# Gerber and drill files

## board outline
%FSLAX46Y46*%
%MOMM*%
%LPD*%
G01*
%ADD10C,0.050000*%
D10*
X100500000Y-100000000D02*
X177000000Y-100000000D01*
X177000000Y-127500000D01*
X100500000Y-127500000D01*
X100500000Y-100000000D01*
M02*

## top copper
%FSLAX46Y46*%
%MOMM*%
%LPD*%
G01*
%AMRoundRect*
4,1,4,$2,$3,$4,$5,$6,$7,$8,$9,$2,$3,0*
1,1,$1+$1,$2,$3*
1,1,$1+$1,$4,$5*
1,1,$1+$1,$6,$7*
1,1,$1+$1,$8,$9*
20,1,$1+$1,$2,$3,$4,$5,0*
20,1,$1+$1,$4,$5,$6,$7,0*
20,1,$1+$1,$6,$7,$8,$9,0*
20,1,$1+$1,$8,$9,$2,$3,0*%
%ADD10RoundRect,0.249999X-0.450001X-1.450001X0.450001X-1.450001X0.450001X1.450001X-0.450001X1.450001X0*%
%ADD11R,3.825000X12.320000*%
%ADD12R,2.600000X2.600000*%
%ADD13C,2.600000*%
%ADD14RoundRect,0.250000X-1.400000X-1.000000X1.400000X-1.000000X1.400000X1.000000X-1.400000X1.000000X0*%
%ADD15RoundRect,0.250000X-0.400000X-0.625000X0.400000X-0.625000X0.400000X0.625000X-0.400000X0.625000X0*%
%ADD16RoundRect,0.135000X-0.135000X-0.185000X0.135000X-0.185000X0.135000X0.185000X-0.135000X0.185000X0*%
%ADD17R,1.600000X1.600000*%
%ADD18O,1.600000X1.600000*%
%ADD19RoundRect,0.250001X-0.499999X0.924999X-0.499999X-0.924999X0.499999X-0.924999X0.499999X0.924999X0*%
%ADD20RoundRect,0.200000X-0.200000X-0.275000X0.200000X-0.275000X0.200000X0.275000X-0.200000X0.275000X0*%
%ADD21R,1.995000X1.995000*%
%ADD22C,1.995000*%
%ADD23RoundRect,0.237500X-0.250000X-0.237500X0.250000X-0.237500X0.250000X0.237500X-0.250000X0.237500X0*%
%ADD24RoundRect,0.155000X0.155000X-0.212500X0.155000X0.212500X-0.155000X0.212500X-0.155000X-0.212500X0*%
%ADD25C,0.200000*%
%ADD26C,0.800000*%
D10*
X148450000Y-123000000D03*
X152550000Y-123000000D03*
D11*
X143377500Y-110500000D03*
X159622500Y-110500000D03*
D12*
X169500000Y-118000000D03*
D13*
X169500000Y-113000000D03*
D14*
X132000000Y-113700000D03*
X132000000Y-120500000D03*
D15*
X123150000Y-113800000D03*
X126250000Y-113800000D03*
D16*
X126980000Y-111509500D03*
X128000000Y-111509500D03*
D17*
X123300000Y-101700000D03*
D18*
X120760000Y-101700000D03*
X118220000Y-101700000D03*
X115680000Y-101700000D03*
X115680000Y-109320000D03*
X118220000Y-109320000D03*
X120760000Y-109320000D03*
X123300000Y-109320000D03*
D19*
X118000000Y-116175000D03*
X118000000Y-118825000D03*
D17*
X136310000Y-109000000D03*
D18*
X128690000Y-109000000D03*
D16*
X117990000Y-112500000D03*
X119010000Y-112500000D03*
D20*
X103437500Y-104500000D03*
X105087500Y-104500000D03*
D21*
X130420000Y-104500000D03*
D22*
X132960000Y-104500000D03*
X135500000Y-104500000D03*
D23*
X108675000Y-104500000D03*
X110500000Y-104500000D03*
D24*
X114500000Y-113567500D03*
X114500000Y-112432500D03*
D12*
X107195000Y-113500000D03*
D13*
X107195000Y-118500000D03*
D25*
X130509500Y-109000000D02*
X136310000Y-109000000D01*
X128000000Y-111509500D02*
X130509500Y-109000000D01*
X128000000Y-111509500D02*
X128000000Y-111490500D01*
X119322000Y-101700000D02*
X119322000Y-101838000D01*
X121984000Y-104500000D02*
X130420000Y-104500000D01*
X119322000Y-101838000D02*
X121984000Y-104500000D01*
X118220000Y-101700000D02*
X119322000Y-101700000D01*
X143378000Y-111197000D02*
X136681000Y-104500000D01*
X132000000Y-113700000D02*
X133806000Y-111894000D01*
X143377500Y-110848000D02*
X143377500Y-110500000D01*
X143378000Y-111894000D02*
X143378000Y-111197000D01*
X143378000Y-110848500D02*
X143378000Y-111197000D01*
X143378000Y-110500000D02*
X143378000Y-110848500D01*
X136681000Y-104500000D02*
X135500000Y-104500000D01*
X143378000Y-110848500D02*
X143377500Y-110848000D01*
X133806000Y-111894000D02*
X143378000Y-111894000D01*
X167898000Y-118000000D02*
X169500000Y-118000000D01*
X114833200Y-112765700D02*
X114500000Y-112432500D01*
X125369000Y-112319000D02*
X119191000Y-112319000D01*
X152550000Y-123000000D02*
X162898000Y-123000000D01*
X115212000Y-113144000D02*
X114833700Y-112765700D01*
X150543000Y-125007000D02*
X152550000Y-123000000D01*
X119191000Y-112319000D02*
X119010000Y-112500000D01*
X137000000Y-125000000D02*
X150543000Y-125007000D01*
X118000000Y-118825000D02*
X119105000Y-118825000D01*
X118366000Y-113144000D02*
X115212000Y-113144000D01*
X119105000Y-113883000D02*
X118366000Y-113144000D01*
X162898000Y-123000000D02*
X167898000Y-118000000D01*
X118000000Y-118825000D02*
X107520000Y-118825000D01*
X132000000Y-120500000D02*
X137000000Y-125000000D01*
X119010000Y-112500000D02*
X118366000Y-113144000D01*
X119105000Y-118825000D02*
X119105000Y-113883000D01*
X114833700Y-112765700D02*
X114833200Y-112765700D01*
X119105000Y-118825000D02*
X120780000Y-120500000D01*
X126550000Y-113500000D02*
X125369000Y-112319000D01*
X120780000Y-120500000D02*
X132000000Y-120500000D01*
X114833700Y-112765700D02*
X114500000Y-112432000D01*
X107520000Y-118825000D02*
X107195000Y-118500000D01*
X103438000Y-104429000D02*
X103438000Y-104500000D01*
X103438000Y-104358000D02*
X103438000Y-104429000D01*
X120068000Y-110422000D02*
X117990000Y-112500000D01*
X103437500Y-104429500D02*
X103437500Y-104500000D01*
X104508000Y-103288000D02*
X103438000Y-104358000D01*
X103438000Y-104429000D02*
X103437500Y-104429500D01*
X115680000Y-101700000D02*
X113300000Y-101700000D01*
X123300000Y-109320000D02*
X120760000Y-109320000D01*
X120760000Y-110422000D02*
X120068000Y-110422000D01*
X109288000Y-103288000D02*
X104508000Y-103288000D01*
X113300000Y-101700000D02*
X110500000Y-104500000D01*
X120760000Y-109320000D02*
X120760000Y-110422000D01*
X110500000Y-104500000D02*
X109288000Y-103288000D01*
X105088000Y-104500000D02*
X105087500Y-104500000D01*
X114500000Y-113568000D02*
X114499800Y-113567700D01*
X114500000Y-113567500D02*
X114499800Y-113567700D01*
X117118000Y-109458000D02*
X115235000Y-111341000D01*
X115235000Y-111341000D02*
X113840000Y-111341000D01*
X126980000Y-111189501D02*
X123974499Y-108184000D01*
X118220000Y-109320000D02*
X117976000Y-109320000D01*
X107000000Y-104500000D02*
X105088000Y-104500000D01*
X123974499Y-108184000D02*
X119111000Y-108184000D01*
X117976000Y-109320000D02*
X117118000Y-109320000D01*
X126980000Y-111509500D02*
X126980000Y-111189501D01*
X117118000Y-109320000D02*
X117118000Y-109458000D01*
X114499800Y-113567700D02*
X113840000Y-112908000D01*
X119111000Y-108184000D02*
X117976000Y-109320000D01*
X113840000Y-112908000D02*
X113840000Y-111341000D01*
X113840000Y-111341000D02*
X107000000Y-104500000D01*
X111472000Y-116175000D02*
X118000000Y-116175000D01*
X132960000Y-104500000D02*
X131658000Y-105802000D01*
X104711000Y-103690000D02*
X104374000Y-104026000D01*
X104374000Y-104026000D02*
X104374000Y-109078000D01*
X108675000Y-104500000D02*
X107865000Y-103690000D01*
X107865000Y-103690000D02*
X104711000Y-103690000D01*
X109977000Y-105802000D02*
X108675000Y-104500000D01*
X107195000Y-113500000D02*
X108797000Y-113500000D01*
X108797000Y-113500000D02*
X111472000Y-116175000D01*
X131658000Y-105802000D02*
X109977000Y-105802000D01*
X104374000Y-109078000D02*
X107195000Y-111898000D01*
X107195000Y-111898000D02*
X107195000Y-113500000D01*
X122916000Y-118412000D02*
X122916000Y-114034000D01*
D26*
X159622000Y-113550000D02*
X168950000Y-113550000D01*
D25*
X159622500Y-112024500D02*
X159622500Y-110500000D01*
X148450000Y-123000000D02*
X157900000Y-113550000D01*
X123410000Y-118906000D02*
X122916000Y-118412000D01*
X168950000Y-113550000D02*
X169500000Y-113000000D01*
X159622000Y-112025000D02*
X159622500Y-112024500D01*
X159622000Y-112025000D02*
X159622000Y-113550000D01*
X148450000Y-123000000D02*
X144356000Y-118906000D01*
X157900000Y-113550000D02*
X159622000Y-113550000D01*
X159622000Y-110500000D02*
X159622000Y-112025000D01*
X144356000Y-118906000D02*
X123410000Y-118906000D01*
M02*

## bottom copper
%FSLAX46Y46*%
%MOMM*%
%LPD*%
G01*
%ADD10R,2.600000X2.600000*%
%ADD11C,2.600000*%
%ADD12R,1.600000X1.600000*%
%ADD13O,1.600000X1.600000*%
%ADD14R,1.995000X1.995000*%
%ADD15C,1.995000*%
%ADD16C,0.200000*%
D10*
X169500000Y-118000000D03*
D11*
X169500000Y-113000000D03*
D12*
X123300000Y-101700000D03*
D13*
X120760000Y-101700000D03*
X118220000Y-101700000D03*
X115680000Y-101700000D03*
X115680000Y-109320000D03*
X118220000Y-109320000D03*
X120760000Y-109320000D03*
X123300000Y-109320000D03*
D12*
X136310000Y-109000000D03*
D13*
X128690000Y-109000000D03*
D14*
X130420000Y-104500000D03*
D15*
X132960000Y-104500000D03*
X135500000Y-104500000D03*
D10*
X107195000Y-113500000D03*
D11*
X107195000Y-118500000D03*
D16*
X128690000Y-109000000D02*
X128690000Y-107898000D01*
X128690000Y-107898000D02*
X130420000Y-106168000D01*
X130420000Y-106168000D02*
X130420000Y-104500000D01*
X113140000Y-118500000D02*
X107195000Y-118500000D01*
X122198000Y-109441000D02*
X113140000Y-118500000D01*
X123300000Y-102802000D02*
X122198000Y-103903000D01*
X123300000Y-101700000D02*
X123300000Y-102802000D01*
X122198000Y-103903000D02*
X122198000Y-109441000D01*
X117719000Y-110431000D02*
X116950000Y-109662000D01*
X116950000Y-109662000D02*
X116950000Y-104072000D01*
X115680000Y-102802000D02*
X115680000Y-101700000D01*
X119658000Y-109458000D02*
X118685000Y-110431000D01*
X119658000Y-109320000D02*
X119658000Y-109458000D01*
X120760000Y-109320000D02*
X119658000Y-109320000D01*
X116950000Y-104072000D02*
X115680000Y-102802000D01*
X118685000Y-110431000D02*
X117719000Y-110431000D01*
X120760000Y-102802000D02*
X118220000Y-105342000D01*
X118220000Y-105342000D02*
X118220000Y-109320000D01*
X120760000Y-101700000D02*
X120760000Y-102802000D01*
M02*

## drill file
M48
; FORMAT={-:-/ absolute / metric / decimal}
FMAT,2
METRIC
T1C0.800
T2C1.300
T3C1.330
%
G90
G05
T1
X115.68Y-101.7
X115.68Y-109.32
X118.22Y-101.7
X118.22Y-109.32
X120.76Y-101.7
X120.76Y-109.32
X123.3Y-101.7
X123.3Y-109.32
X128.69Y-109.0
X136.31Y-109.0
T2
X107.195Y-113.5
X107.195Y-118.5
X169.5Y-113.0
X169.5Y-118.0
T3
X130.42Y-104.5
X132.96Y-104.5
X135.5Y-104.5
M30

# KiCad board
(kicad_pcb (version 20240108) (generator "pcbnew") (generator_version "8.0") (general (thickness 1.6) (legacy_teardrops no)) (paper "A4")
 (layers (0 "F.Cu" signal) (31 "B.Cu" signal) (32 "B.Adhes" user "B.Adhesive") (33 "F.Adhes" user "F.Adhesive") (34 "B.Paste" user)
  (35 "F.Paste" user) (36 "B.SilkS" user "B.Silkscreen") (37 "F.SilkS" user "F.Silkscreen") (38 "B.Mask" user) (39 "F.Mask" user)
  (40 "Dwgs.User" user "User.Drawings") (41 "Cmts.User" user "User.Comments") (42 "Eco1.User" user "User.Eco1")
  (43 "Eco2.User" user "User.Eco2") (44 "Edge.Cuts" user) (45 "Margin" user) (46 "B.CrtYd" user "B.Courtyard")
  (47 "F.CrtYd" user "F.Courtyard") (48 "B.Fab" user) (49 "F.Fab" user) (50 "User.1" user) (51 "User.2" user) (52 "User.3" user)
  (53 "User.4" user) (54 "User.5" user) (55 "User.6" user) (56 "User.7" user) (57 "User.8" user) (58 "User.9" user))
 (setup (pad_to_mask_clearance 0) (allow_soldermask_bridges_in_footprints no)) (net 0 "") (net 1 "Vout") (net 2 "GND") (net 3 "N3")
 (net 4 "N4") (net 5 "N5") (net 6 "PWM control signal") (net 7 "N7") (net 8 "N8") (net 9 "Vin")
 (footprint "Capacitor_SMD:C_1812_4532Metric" (layer "F.Cu") (at 150.5 123)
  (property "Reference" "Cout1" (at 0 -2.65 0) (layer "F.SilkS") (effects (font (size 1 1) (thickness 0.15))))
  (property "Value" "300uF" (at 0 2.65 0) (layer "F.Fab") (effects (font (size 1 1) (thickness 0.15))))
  (pad "1" smd roundrect (at -2.05 0) (size 1.4 3.4) (layers "F.Cu" "F.Paste" "F.Mask") (roundrect_rratio 0.178571) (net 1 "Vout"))
  (pad "2" smd roundrect (at 2.05 0) (size 1.4 3.4) (layers "F.Cu" "F.Paste" "F.Mask") (roundrect_rratio 0.178571) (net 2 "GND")))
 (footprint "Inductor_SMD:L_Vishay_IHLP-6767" (layer "F.Cu") (at 151.5 110.5)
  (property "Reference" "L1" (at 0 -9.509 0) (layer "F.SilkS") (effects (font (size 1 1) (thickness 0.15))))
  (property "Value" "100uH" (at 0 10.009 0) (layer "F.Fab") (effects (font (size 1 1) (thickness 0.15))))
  (pad "1" smd rect (at -8.1225 0) (size 3.825 12.32) (layers "F.Cu" "F.Paste" "F.Mask") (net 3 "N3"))
  (pad "2" smd rect (at 8.1225 0) (size 3.825 12.32) (layers "F.Cu" "F.Paste" "F.Mask") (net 1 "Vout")))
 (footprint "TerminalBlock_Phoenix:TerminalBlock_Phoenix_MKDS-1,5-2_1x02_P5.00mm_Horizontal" (layer "F.Cu") (at 169.5 118 90)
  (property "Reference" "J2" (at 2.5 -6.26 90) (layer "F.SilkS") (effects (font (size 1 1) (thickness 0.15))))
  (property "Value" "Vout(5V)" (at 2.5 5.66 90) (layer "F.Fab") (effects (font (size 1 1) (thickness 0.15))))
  (pad "1" thru_hole rect (at 0 0 90) (size 2.6 2.6) (drill 1.3) (layers "*.Cu" "*.Mask") (remove_unused_layers no) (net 2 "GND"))
  (pad "2" thru_hole circle (at 5 0 90) (size 2.6 2.6) (drill 1.3) (layers "*.Cu" "*.Mask") (remove_unused_layers no) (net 1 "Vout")))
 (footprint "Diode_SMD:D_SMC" (layer "F.Cu") (at 132 117.1 -90)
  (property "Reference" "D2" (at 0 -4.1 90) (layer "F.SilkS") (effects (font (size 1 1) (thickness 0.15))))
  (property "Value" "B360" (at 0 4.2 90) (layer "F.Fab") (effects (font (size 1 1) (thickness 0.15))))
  (pad "1" smd roundrect (at -3.4 0) (size 3.3 2.5) (layers "F.Cu" "F.Paste" "F.Mask") (roundrect_rratio 0.1) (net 3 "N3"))
  (pad "2" smd roundrect (at 3.4 0) (size 3.3 2.5) (layers "F.Cu" "F.Paste" "F.Mask") (roundrect_rratio 0.1) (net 2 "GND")))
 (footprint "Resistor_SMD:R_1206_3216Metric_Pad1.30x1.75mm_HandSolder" (layer "F.Cu") (at 124.7 113.8)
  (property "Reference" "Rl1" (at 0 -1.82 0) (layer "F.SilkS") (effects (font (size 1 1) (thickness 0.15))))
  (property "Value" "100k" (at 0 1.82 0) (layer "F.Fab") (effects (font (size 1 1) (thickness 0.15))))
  (pad "1" smd roundrect (at -1.55 0) (size 1.3 1.75) (layers "F.Cu" "F.Paste" "F.Mask") (roundrect_rratio 0.192308) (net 1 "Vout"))
  (pad "2" smd roundrect (at 1.55 0) (size 1.3 1.75) (layers "F.Cu" "F.Paste" "F.Mask") (roundrect_rratio 0.192308) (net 2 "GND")))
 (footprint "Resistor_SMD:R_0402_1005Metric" (layer "F.Cu") (at 127.49 111.5095)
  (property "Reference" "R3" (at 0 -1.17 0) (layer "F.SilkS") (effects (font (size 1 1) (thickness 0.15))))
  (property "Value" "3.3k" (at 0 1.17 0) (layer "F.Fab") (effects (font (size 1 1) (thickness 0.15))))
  (pad "1" smd roundrect (at -0.51 0) (size 0.54 0.64) (layers "F.Cu" "F.Paste" "F.Mask") (roundrect_rratio 0.25) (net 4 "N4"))
  (pad "2" smd roundrect (at 0.51 0) (size 0.54 0.64) (layers "F.Cu" "F.Paste" "F.Mask") (roundrect_rratio 0.25) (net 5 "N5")))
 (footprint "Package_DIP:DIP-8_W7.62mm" (layer "F.Cu") (at 123.3 101.7 -90)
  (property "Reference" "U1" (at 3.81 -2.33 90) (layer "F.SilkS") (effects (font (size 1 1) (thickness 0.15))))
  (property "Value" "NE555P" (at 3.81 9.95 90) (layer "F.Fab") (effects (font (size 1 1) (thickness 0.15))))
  (pad "1" thru_hole rect (at 0 0 270) (size 1.6 1.6) (drill 0.8) (layers "*.Cu" "*.Mask") (remove_unused_layers no) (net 2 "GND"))
  (pad "2" thru_hole oval (at 0 2.54 270) (size 1.6 1.6) (drill 0.8) (layers "*.Cu" "*.Mask") (remove_unused_layers no) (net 4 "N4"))
  (pad "3" thru_hole oval (at 0 5.08 270) (size 1.6 1.6) (drill 0.8) (layers "*.Cu" "*.Mask") (remove_unused_layers no)
   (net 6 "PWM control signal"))
  (pad "4" thru_hole oval (at 0 7.62 270) (size 1.6 1.6) (drill 0.8) (layers "*.Cu" "*.Mask") (remove_unused_layers no) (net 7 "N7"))
  (pad "5" thru_hole oval (at 7.62 7.62 270) (size 1.6 1.6) (drill 0.8) (layers "*.Cu" "*.Mask") (remove_unused_layers no) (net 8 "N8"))
  (pad "6" thru_hole oval (at 7.62 5.08 270) (size 1.6 1.6) (drill 0.8) (layers "*.Cu" "*.Mask") (remove_unused_layers no) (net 4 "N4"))
  (pad "7" thru_hole oval (at 7.62 2.54 270) (size 1.6 1.6) (drill 0.8) (layers "*.Cu" "*.Mask") (remove_unused_layers no) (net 7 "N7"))
  (pad "8" thru_hole oval (at 7.62 0 270) (size 1.6 1.6) (drill 0.8) (layers "*.Cu" "*.Mask") (remove_unused_layers no) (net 7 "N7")))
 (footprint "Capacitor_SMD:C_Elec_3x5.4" (layer "F.Cu") (at 118 117.5 -90)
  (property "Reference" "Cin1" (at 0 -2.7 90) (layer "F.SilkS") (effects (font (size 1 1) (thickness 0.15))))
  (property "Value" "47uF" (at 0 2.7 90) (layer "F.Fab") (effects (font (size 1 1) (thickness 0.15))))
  (pad "1" smd roundrect (at -1.325 0 270) (size 2.35 1.5) (layers "F.Cu" "F.Paste" "F.Mask") (roundrect_rratio 0.166667) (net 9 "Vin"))
  (pad "2" smd roundrect (at 1.325 0 270) (size 2.35 1.5) (layers "F.Cu" "F.Paste" "F.Mask") (roundrect_rratio 0.166667) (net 2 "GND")))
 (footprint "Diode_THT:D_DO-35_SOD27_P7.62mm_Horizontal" (layer "F.Cu") (at 136.31 109 180)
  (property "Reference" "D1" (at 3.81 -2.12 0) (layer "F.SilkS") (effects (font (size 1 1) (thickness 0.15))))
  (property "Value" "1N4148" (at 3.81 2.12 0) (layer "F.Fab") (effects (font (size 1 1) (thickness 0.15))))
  (pad "1" thru_hole rect (at 0 0 180) (size 1.6 1.6) (drill 0.8) (layers "*.Cu" "*.Mask") (remove_unused_layers no) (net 5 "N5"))
  (pad "2" thru_hole oval (at 7.62 0 180) (size 1.6 1.6) (drill 0.8) (layers "*.Cu" "*.Mask") (remove_unused_layers no)
   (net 6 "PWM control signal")))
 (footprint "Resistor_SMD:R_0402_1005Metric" (layer "F.Cu") (at 118.5 112.5)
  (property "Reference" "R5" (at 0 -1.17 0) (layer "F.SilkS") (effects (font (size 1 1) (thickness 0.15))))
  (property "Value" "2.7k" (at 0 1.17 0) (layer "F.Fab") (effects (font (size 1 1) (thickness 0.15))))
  (pad "1" smd roundrect (at -0.51 0) (size 0.54 0.64) (layers "F.Cu" "F.Paste" "F.Mask") (roundrect_rratio 0.25) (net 7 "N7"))
  (pad "2" smd roundrect (at 0.51 0) (size 0.54 0.64) (layers "F.Cu" "F.Paste" "F.Mask") (roundrect_rratio 0.25) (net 2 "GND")))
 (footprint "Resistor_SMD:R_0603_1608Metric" (layer "F.Cu") (at 104.2625 104.5)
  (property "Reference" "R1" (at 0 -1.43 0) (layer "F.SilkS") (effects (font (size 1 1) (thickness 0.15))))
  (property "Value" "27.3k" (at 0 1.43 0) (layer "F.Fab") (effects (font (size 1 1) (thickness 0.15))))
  (pad "1" smd roundrect (at -0.825 0) (size 0.8 0.95) (layers "F.Cu" "F.Paste" "F.Mask") (roundrect_rratio 0.25) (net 7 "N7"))
  (pad "2" smd roundrect (at 0.825 0) (size 0.8 0.95) (layers "F.Cu" "F.Paste" "F.Mask") (roundrect_rratio 0.25) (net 4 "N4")))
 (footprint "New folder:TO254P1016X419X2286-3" (layer "F.Cu") (at 132.96 104.5)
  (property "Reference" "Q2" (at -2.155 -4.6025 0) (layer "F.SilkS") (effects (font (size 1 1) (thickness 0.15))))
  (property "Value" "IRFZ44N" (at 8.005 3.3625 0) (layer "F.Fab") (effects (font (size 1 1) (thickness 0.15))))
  (pad "1" thru_hole rect (at -2.54 0) (size 1.995 1.995) (drill 1.33) (layers "*.Cu" "*.Mask") (remove_unused_layers no)
   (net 6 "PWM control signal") (solder_mask_margin 0.102))
  (pad "2" thru_hole circle (at 0 0) (size 1.995 1.995) (drill 1.33) (layers "*.Cu" "*.Mask") (remove_unused_layers no) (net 9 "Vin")
   (solder_mask_margin 0.102))
  (pad "3" thru_hole circle (at 2.54 0) (size 1.995 1.995) (drill 1.33) (layers "*.Cu" "*.Mask") (remove_unused_layers no) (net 3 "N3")
   (solder_mask_margin 0.102)))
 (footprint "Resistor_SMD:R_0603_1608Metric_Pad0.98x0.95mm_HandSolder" (layer "F.Cu") (at 109.5875 104.5)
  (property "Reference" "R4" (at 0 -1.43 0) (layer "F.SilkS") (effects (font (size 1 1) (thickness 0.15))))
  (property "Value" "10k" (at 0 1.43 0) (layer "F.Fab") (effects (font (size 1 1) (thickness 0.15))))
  (pad "1" smd roundrect (at -0.9125 0) (size 0.975 0.95) (layers "F.Cu" "F.Paste" "F.Mask") (roundrect_rratio 0.25) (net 9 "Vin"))
  (pad "2" smd roundrect (at 0.9125 0) (size 0.975 0.95) (layers "F.Cu" "F.Paste" "F.Mask") (roundrect_rratio 0.25) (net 7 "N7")))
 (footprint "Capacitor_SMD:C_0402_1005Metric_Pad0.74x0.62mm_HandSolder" (layer "F.Cu") (at 114.5 113 90)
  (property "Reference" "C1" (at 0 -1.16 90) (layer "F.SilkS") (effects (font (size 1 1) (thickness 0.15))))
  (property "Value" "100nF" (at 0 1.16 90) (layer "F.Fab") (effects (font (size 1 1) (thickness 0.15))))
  (pad "1" smd roundrect (at -0.5675 0 90) (size 0.735 0.62) (layers "F.Cu" "F.Paste" "F.Mask") (roundrect_rratio 0.25) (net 4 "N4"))
  (pad "2" smd roundrect (at 0.5675 0 90) (size 0.735 0.62) (layers "F.Cu" "F.Paste" "F.Mask") (roundrect_rratio 0.25) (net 2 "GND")))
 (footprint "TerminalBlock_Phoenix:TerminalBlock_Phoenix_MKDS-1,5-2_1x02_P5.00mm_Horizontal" (layer "F.Cu") (at 107.195 113.5 -90)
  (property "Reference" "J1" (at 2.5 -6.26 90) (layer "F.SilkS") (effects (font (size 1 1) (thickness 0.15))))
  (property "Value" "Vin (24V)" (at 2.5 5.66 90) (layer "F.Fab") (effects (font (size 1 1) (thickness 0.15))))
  (pad "1" thru_hole rect (at 0 0 270) (size 2.6 2.6) (drill 1.3) (layers "*.Cu" "*.Mask") (remove_unused_layers no) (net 9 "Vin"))
  (pad "2" thru_hole circle (at 5 0 270) (size 2.6 2.6) (drill 1.3) (layers "*.Cu" "*.Mask") (remove_unused_layers no) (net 2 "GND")))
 (gr_rect (start 100.5 100) (end 177 127.5) (stroke (width 0.05) (type default)) (fill none) (layer "Edge.Cuts"))
 (segment (start 130.5095 109) (end 136.31 109) (width 0.2) (layer "F.Cu") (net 5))
 (segment (start 128 111.5095) (end 130.5095 109) (width 0.2) (layer "F.Cu") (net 5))
 (segment (start 128 111.5095) (end 128 111.4905) (width 0.2) (layer "F.Cu") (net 5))
 (segment (start 119.322 101.7) (end 119.322 101.838) (width 0.2) (layer "F.Cu") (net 6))
 (segment (start 121.984 104.5) (end 130.42 104.5) (width 0.2) (layer "F.Cu") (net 6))
 (segment (start 119.322 101.838) (end 121.984 104.5) (width 0.2) (layer "F.Cu") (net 6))
 (segment (start 118.22 101.7) (end 119.322 101.7) (width 0.2) (layer "F.Cu") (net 6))
 (segment (start 128.69 109) (end 128.69 107.898) (width 0.2) (layer "B.Cu") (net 6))
 (segment (start 128.69 107.898) (end 130.42 106.168) (width 0.2) (layer "B.Cu") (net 6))
 (segment (start 130.42 106.168) (end 130.42 104.5) (width 0.2) (layer "B.Cu") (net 6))
 (segment (start 143.378 111.197) (end 136.681 104.5) (width 0.2) (layer "F.Cu") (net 3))
 (segment (start 132 113.7) (end 133.806 111.894) (width 0.2) (layer "F.Cu") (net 3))
 (segment (start 143.3775 110.848) (end 143.3775 110.5) (width 0.2) (layer "F.Cu") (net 3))
 (segment (start 143.378 111.894) (end 143.378 111.197) (width 0.2) (layer "F.Cu") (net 3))
 (segment (start 143.378 110.8485) (end 143.378 111.197) (width 0.2) (layer "F.Cu") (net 3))
 (segment (start 143.378 110.5) (end 143.378 110.8485) (width 0.2) (layer "F.Cu") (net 3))
 (segment (start 136.681 104.5) (end 135.5 104.5) (width 0.2) (layer "F.Cu") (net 3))
 (segment (start 143.378 110.8485) (end 143.3775 110.848) (width 0.2) (layer "F.Cu") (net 3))
 (segment (start 133.806 111.894) (end 143.378 111.894) (width 0.2) (layer "F.Cu") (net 3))
 (segment (start 167.898 118) (end 169.5 118) (width 0.2) (layer "F.Cu") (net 2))
 (segment (start 114.8332 112.7657) (end 114.5 112.4325) (width 0.2) (layer "F.Cu") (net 2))
 (segment (start 125.369 112.319) (end 119.191 112.319) (width 0.2) (layer "F.Cu") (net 2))
 (segment (start 152.55 123) (end 162.898 123) (width 0.2) (layer "F.Cu") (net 2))
 (segment (start 115.212 113.144) (end 114.8337 112.7657) (width 0.2) (layer "F.Cu") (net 2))
 (segment (start 150.543 125.007) (end 152.55 123) (width 0.2) (layer "F.Cu") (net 2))
 (segment (start 119.191 112.319) (end 119.01 112.5) (width 0.2) (layer "F.Cu") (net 2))
 (segment (start 137 125) (end 150.543 125.007) (width 0.2) (layer "F.Cu") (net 2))
 (segment (start 118 118.825) (end 119.105 118.825) (width 0.2) (layer "F.Cu") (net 2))
 (segment (start 118.366 113.144) (end 115.212 113.144) (width 0.2) (layer "F.Cu") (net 2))
 (segment (start 119.105 113.883) (end 118.366 113.144) (width 0.2) (layer "F.Cu") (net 2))
 (segment (start 162.898 123) (end 167.898 118) (width 0.2) (layer "F.Cu") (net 2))
 (segment (start 118 118.825) (end 107.52 118.825) (width 0.2) (layer "F.Cu") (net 2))
 (segment (start 132 120.5) (end 137 125) (width 0.2) (layer "F.Cu") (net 2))
 (segment (start 119.01 112.5) (end 118.366 113.144) (width 0.2) (layer "F.Cu") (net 2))
 (segment (start 119.105 118.825) (end 119.105 113.883) (width 0.2) (layer "F.Cu") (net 2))
 (segment (start 114.8337 112.7657) (end 114.8332 112.7657) (width 0.2) (layer "F.Cu") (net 2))
 (segment (start 119.105 118.825) (end 120.78 120.5) (width 0.2) (layer "F.Cu") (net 2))
 (segment (start 126.55 113.5) (end 125.369 112.319) (width 0.2) (layer "F.Cu") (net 2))
 (segment (start 120.78 120.5) (end 132 120.5) (width 0.2) (layer "F.Cu") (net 2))
 (segment (start 114.8337 112.7657) (end 114.5 112.432) (width 0.2) (layer "F.Cu") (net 2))
 (segment (start 107.52 118.825) (end 107.195 118.5) (width 0.2) (layer "F.Cu") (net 2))
 (segment (start 113.14 118.5) (end 107.195 118.5) (width 0.2) (layer "B.Cu") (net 2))
 (segment (start 122.198 109.441) (end 113.14 118.5) (width 0.2) (layer "B.Cu") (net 2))
 (segment (start 123.3 102.802) (end 122.198 103.903) (width 0.2) (layer "B.Cu") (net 2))
 (segment (start 123.3 101.7) (end 123.3 102.802) (width 0.2) (layer "B.Cu") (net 2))
 (segment (start 122.198 103.903) (end 122.198 109.441) (width 0.2) (layer "B.Cu") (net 2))
 (segment (start 103.438 104.429) (end 103.438 104.5) (width 0.2) (layer "F.Cu") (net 7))
 (segment (start 103.438 104.358) (end 103.438 104.429) (width 0.2) (layer "F.Cu") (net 7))
 (segment (start 120.068 110.422) (end 117.99 112.5) (width 0.2) (layer "F.Cu") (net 7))
 (segment (start 103.4375 104.4295) (end 103.4375 104.5) (width 0.2) (layer "F.Cu") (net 7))
 (segment (start 104.508 103.288) (end 103.438 104.358) (width 0.2) (layer "F.Cu") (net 7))
 (segment (start 103.438 104.429) (end 103.4375 104.4295) (width 0.2) (layer "F.Cu") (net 7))
 (segment (start 115.68 101.7) (end 113.3 101.7) (width 0.2) (layer "F.Cu") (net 7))
 (segment (start 123.3 109.32) (end 120.76 109.32) (width 0.2) (layer "F.Cu") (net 7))
 (segment (start 120.76 110.422) (end 120.068 110.422) (width 0.2) (layer "F.Cu") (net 7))
 (segment (start 109.288 103.288) (end 104.508 103.288) (width 0.2) (layer "F.Cu") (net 7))
 (segment (start 113.3 101.7) (end 110.5 104.5) (width 0.2) (layer "F.Cu") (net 7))
 (segment (start 120.76 109.32) (end 120.76 110.422) (width 0.2) (layer "F.Cu") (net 7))
 (segment (start 110.5 104.5) (end 109.288 103.288) (width 0.2) (layer "F.Cu") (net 7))
 (segment (start 117.719 110.431) (end 116.95 109.662) (width 0.2) (layer "B.Cu") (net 7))
 (segment (start 116.95 109.662) (end 116.95 104.072) (width 0.2) (layer "B.Cu") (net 7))
 (segment (start 115.68 102.802) (end 115.68 101.7) (width 0.2) (layer "B.Cu") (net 7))
 (segment (start 119.658 109.458) (end 118.685 110.431) (width 0.2) (layer "B.Cu") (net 7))
 (segment (start 119.658 109.32) (end 119.658 109.458) (width 0.2) (layer "B.Cu") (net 7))
 (segment (start 120.76 109.32) (end 119.658 109.32) (width 0.2) (layer "B.Cu") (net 7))
 (segment (start 116.95 104.072) (end 115.68 102.802) (width 0.2) (layer "B.Cu") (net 7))
 (segment (start 118.685 110.431) (end 117.719 110.431) (width 0.2) (layer "B.Cu") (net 7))
 (segment (start 105.088 104.5) (end 105.0875 104.5) (width 0.2) (layer "F.Cu") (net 4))
 (segment (start 114.5 113.568) (end 114.4998 113.5677) (width 0.2) (layer "F.Cu") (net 4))
 (segment (start 114.5 113.5675) (end 114.4998 113.5677) (width 0.2) (layer "F.Cu") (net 4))
 (segment (start 117.118 109.458) (end 115.235 111.341) (width 0.2) (layer "F.Cu") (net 4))
 (segment (start 115.235 111.341) (end 113.84 111.341) (width 0.2) (layer "F.Cu") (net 4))
 (segment (start 126.98 111.189501) (end 123.974499 108.184) (width 0.2) (layer "F.Cu") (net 4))
 (segment (start 118.22 109.32) (end 117.976 109.32) (width 0.2) (layer "F.Cu") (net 4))
 (segment (start 107 104.5) (end 105.088 104.5) (width 0.2) (layer "F.Cu") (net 4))
 (segment (start 123.974499 108.184) (end 119.111 108.184) (width 0.2) (layer "F.Cu") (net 4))
 (segment (start 117.976 109.32) (end 117.118 109.32) (width 0.2) (layer "F.Cu") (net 4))
 (segment (start 126.98 111.5095) (end 126.98 111.189501) (width 0.2) (layer "F.Cu") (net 4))
 (segment (start 117.118 109.32) (end 117.118 109.458) (width 0.2) (layer "F.Cu") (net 4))
 (segment (start 114.4998 113.5677) (end 113.84 112.908) (width 0.2) (layer "F.Cu") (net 4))
 (segment (start 119.111 108.184) (end 117.976 109.32) (width 0.2) (layer "F.Cu") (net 4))
 (segment (start 113.84 112.908) (end 113.84 111.341) (width 0.2) (layer "F.Cu") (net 4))
 (segment (start 113.84 111.341) (end 107 104.5) (width 0.2) (layer "F.Cu") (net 4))
 (segment (start 120.76 102.802) (end 118.22 105.342) (width 0.2) (layer "B.Cu") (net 4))
 (segment (start 118.22 105.342) (end 118.22 109.32) (width 0.2) (layer "B.Cu") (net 4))
 (segment (start 120.76 101.7) (end 120.76 102.802) (width 0.2) (layer "B.Cu") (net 4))
 (segment (start 111.472 116.175) (end 118 116.175) (width 0.2) (layer "F.Cu") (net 9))
 (segment (start 132.96 104.5) (end 131.658 105.802) (width 0.2) (layer "F.Cu") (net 9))
 (segment (start 104.711 103.69) (end 104.374 104.026) (width 0.2) (layer "F.Cu") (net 9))
 (segment (start 104.374 104.026) (end 104.374 109.078) (width 0.2) (layer "F.Cu") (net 9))
 (segment (start 108.675 104.5) (end 107.865 103.69) (width 0.2) (layer "F.Cu") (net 9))
 (segment (start 107.865 103.69) (end 104.711 103.69) (width 0.2) (layer "F.Cu") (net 9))
 (segment (start 109.977 105.802) (end 108.675 104.5) (width 0.2) (layer "F.Cu") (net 9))
 (segment (start 107.195 113.5) (end 108.797 113.5) (width 0.2) (layer "F.Cu") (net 9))
 (segment (start 108.797 113.5) (end 111.472 116.175) (width 0.2) (layer "F.Cu") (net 9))
 (segment (start 131.658 105.802) (end 109.977 105.802) (width 0.2) (layer "F.Cu") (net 9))
 (segment (start 104.374 109.078) (end 107.195 111.898) (width 0.2) (layer "F.Cu") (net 9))
 (segment (start 107.195 111.898) (end 107.195 113.5) (width 0.2) (layer "F.Cu") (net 9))
 (segment (start 122.916 118.412) (end 122.916 114.034) (width 0.2) (layer "F.Cu") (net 1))
 (segment (start 159.622 113.55) (end 168.95 113.55) (width 0.8) (layer "F.Cu") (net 1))
 (segment (start 159.6225 112.0245) (end 159.6225 110.5) (width 0.2) (layer "F.Cu") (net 1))
 (segment (start 148.45 123) (end 157.9 113.55) (width 0.2) (layer "F.Cu") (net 1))
 (segment (start 123.41 118.906) (end 122.916 118.412) (width 0.2) (layer "F.Cu") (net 1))
 (segment (start 168.95 113.55) (end 169.5 113) (width 0.2) (layer "F.Cu") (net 1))
 (segment (start 159.622 112.025) (end 159.6225 112.0245) (width 0.2) (layer "F.Cu") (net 1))
 (segment (start 159.622 112.025) (end 159.622 113.55) (width 0.2) (layer "F.Cu") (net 1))
 (segment (start 148.45 123) (end 144.356 118.906) (width 0.2) (layer "F.Cu") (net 1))
 (segment (start 157.9 113.55) (end 159.622 113.55) (width 0.2) (layer "F.Cu") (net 1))
 (segment (start 159.622 110.5) (end 159.622 112.025) (width 0.2) (layer "F.Cu") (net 1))
 (segment (start 144.356 118.906) (end 123.41 118.906) (width 0.2) (layer "F.Cu") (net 1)))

